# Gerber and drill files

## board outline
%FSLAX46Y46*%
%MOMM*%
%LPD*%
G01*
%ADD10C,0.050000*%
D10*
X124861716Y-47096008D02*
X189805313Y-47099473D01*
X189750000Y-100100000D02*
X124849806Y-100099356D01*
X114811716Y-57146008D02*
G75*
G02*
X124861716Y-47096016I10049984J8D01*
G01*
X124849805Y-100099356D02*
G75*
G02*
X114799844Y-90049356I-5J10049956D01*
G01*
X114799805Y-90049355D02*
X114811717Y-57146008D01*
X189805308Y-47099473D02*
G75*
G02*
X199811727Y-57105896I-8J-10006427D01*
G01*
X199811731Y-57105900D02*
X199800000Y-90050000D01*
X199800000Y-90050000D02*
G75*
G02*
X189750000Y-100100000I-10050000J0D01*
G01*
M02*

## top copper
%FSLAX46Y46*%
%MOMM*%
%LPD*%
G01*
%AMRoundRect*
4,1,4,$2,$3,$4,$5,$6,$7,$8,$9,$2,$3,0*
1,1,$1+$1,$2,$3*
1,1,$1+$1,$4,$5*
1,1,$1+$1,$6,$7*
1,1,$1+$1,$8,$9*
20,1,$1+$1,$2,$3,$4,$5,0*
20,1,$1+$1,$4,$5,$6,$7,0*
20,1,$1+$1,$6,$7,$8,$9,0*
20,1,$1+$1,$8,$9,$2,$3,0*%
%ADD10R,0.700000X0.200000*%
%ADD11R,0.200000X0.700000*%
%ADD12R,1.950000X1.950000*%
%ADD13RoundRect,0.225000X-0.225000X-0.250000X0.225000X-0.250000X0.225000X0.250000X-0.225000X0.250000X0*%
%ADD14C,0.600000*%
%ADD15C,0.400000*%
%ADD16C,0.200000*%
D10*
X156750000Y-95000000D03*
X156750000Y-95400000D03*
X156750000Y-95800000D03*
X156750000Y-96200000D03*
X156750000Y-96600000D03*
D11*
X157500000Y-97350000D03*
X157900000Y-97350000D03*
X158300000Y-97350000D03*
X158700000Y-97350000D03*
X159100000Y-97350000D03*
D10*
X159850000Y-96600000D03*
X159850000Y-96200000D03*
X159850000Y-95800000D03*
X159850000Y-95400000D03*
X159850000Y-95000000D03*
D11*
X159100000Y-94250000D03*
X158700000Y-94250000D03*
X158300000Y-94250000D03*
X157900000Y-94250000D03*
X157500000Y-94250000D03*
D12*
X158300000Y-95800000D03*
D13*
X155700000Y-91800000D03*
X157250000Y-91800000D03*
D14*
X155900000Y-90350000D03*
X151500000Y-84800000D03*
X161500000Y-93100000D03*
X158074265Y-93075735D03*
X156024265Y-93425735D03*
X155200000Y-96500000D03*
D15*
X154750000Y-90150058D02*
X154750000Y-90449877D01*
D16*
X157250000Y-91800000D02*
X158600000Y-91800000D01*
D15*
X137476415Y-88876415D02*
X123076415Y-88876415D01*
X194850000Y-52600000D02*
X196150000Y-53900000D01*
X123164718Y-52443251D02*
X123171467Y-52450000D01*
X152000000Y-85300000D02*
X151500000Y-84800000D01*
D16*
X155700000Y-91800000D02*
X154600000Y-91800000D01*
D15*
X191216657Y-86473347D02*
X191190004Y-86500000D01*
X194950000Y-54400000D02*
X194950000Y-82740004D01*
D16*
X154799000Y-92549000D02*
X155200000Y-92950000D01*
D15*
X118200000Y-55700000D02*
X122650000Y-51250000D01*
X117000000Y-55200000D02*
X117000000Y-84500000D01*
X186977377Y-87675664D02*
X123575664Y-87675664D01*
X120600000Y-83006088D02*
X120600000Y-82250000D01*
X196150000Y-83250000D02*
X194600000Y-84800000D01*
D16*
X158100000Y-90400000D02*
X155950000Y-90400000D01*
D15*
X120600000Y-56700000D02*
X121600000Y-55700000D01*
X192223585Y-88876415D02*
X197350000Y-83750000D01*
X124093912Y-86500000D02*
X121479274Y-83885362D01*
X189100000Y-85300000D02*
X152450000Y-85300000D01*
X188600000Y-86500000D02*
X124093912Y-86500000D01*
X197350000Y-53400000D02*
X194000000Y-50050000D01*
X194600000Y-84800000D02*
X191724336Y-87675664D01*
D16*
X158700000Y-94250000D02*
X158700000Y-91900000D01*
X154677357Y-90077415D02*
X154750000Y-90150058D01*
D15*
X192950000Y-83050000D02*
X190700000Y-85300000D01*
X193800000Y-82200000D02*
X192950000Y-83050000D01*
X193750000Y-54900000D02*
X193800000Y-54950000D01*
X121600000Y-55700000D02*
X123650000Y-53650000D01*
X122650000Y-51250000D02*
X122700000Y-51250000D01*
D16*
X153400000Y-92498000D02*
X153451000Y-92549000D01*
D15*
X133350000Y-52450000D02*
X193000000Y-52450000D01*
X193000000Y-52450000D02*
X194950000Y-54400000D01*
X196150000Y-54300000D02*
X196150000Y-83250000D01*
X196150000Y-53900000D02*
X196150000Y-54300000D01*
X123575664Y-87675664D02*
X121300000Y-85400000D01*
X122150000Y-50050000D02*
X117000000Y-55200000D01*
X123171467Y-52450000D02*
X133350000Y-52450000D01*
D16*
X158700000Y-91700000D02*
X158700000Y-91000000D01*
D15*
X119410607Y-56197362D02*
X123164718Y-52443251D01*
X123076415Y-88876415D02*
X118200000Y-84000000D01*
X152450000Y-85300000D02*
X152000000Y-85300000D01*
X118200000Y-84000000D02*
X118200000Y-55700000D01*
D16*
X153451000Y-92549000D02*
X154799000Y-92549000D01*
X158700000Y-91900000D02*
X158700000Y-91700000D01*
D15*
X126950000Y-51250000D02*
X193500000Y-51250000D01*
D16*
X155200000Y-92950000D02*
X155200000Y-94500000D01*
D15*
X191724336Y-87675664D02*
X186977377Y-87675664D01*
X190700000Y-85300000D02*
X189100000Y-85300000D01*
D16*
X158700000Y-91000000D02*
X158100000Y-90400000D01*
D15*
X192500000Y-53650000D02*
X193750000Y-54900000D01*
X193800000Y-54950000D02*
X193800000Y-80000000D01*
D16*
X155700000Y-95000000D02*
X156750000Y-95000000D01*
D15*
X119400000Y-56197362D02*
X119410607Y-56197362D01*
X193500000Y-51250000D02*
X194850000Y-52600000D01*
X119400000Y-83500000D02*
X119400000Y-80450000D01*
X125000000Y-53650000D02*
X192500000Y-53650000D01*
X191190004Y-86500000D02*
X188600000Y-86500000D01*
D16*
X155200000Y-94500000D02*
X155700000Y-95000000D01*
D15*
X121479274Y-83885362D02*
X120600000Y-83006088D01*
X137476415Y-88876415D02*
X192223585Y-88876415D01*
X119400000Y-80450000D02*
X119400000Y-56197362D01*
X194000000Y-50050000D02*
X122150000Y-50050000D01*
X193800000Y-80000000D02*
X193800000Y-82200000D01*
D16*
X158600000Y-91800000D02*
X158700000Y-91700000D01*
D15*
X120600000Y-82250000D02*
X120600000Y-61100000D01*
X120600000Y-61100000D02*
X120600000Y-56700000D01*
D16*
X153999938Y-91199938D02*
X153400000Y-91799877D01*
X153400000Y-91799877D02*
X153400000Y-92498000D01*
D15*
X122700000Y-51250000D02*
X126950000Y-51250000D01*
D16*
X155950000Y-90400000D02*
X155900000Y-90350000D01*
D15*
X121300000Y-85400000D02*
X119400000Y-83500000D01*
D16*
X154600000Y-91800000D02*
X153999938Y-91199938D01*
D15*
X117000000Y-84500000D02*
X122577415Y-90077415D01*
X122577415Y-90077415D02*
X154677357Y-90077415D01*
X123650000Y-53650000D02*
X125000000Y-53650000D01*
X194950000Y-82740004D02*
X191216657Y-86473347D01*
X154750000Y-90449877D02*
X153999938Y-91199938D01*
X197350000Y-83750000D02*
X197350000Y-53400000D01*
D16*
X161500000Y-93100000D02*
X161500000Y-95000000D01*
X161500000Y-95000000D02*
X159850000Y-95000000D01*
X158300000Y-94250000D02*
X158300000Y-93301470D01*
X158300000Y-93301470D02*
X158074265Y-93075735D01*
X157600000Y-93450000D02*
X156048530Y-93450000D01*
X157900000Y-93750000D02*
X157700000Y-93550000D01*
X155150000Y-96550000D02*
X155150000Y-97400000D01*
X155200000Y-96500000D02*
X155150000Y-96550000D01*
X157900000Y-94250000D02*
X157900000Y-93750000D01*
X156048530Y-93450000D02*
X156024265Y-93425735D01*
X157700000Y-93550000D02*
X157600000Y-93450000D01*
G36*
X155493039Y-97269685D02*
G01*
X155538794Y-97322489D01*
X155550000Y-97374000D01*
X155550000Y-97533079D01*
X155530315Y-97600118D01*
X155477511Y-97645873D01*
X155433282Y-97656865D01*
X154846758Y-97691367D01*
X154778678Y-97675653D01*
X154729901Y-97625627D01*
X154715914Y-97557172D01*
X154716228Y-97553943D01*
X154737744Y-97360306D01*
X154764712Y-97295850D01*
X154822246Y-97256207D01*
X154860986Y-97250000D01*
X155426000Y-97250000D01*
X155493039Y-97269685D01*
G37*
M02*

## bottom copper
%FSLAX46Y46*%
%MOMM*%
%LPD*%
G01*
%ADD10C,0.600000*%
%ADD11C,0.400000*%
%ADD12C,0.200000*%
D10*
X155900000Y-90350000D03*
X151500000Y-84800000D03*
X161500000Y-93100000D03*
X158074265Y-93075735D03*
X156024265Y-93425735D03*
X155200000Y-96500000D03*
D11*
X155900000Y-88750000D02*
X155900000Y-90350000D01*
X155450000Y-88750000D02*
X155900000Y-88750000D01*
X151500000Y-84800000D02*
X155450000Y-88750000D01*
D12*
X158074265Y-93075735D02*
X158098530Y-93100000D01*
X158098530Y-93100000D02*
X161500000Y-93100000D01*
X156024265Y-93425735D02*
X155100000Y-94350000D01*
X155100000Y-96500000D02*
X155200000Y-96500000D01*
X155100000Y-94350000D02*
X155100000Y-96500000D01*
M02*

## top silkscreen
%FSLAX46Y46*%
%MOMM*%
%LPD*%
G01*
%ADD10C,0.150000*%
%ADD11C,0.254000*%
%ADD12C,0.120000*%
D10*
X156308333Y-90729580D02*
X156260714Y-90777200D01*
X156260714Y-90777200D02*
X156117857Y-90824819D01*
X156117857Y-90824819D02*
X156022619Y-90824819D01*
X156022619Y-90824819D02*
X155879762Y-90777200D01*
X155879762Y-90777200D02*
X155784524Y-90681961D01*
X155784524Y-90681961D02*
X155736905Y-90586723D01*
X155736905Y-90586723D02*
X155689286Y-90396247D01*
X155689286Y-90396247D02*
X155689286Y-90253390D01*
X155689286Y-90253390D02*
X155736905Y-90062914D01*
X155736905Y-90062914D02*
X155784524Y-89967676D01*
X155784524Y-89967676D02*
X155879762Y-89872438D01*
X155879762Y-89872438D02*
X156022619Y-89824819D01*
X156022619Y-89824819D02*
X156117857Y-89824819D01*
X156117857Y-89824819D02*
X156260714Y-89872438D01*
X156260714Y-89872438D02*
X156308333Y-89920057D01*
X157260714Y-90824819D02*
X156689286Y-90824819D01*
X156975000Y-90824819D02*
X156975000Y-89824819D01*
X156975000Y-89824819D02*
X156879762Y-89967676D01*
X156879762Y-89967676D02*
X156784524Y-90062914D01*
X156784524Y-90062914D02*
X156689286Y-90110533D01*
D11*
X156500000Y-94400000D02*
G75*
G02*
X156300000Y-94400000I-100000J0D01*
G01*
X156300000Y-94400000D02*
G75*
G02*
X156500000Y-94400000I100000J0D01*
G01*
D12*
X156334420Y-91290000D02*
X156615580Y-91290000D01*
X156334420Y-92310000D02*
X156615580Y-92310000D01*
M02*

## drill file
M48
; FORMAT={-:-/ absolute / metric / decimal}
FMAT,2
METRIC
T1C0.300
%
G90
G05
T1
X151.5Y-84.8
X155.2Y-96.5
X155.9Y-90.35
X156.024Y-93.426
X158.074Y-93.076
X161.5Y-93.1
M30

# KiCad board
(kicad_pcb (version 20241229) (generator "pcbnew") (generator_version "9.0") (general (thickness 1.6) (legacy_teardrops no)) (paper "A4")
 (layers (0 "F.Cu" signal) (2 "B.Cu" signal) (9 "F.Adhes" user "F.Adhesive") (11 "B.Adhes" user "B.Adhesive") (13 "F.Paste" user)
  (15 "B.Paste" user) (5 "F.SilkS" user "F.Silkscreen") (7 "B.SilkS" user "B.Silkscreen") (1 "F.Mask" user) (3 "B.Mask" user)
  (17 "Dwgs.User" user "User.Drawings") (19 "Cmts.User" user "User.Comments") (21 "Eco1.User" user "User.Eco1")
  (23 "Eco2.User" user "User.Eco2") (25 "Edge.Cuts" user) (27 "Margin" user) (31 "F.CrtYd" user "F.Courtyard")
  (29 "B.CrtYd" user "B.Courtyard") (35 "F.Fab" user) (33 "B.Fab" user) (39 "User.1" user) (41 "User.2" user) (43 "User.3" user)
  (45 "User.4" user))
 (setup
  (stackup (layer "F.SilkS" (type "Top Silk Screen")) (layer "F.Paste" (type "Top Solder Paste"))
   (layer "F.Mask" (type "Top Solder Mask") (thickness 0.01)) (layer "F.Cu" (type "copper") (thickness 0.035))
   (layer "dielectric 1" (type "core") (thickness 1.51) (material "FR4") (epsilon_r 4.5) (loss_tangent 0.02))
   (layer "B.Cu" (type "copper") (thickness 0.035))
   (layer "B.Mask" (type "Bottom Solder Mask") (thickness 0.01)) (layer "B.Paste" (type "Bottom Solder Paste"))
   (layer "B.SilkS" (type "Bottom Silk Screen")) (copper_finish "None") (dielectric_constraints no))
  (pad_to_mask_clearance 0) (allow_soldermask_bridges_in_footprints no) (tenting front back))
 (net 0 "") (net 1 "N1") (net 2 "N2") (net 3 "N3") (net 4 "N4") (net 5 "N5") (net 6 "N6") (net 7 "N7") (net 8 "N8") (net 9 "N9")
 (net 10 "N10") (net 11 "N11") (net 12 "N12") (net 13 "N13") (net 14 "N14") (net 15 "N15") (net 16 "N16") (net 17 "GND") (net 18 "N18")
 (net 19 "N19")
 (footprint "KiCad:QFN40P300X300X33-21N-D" (layer "F.Cu") (at 158.3 95.8)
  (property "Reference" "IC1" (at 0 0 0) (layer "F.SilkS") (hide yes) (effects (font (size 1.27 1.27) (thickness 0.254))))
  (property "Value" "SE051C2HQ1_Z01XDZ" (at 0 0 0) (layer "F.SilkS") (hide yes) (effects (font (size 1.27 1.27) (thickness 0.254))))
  (fp_circle (center -1.9 -1.4) (end -1.8 -1.4) (stroke (width 0.254) (type solid)) (fill no) (layer "F.SilkS"))
  (pad "1" smd rect (at -1.55 -0.8 90) (size 0.2 0.7) (layers "F.Cu" "F.Mask" "F.Paste") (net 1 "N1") (solder_mask_margin 0.04)
   (thermal_bridge_angle 45))
  (pad "2" smd rect (at -1.55 -0.4 90) (size 0.2 0.7) (layers "F.Cu" "F.Mask" "F.Paste") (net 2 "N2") (solder_mask_margin 0.04)
   (thermal_bridge_angle 45))
  (pad "3" smd rect (at -1.55 0 90) (size 0.2 0.7) (layers "F.Cu" "F.Mask" "F.Paste") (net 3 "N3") (solder_mask_margin 0.04)
   (thermal_bridge_angle 45))
  (pad "4" smd rect (at -1.55 0.4 90) (size 0.2 0.7) (layers "F.Cu" "F.Mask" "F.Paste") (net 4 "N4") (solder_mask_margin 0.04)
   (thermal_bridge_angle 45))
  (pad "5" smd rect (at -1.55 0.8 90) (size 0.2 0.7) (layers "F.Cu" "F.Mask" "F.Paste") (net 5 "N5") (solder_mask_margin 0.04)
   (thermal_bridge_angle 45))
  (pad "6" smd rect (at -0.8 1.55) (size 0.2 0.7) (layers "F.Cu" "F.Mask" "F.Paste") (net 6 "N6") (solder_mask_margin 0.04)
   (thermal_bridge_angle 45))
  (pad "7" smd rect (at -0.4 1.55) (size 0.2 0.7) (layers "F.Cu" "F.Mask" "F.Paste") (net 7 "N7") (solder_mask_margin 0.04)
   (thermal_bridge_angle 45))
  (pad "8" smd rect (at 0 1.55) (size 0.2 0.7) (layers "F.Cu" "F.Mask" "F.Paste") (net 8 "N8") (solder_mask_margin 0.04)
   (thermal_bridge_angle 45))
  (pad "9" smd rect (at 0.4 1.55) (size 0.2 0.7) (layers "F.Cu" "F.Mask" "F.Paste") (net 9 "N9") (solder_mask_margin 0.04)
   (thermal_bridge_angle 45))
  (pad "10" smd rect (at 0.8 1.55) (size 0.2 0.7) (layers "F.Cu" "F.Mask" "F.Paste") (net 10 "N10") (solder_mask_margin 0.04)
   (thermal_bridge_angle 45))
  (pad "11" smd rect (at 1.55 0.8 90) (size 0.2 0.7) (layers "F.Cu" "F.Mask" "F.Paste") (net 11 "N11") (solder_mask_margin 0.04)
   (thermal_bridge_angle 45))
  (pad "12" smd rect (at 1.55 0.4 90) (size 0.2 0.7) (layers "F.Cu" "F.Mask" "F.Paste") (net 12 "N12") (solder_mask_margin 0.04)
   (thermal_bridge_angle 45))
  (pad "13" smd rect (at 1.55 0 90) (size 0.2 0.7) (layers "F.Cu" "F.Mask" "F.Paste") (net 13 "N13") (solder_mask_margin 0.04)
   (thermal_bridge_angle 45))
  (pad "14" smd rect (at 1.55 -0.4 90) (size 0.2 0.7) (layers "F.Cu" "F.Mask" "F.Paste") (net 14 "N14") (solder_mask_margin 0.04)
   (thermal_bridge_angle 45))
  (pad "15" smd rect (at 1.55 -0.8 90) (size 0.2 0.7) (layers "F.Cu" "F.Mask" "F.Paste") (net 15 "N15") (solder_mask_margin 0.04)
   (thermal_bridge_angle 45))
  (pad "16" smd rect (at 0.8 -1.55) (size 0.2 0.7) (layers "F.Cu" "F.Mask" "F.Paste") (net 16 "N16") (solder_mask_margin 0.04)
   (thermal_bridge_angle 45))
  (pad "17" smd rect (at 0.4 -1.55) (size 0.2 0.7) (layers "F.Cu" "F.Mask" "F.Paste") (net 1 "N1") (solder_mask_margin 0.04)
   (thermal_bridge_angle 45))
  (pad "18" smd rect (at 0 -1.55) (size 0.2 0.7) (layers "F.Cu" "F.Mask" "F.Paste") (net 15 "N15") (solder_mask_margin 0.04)
   (thermal_bridge_angle 45))
  (pad "19" smd rect (at -0.4 -1.55) (size 0.2 0.7) (layers "F.Cu" "F.Mask" "F.Paste") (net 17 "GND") (solder_mask_margin 0.04)
   (thermal_bridge_angle 45))
  (pad "20" smd rect (at -0.8 -1.55) (size 0.2 0.7) (layers "F.Cu" "F.Mask" "F.Paste") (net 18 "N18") (solder_mask_margin 0.04)
   (thermal_bridge_angle 45))
  (pad "21" smd rect (at 0 0) (size 1.95 1.95) (layers "F.Cu" "F.Mask" "F.Paste") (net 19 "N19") (thermal_bridge_angle 45)))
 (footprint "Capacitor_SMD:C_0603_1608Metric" (layer "F.Cu") (at 156.475 91.8)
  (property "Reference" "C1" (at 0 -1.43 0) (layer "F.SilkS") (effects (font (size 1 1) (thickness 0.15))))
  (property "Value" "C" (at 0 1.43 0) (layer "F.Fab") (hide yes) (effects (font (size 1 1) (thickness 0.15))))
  (fp_line (start -0.14058 -0.51) (end 0.14058 -0.51) (stroke (width 0.12) (type solid)) (layer "F.SilkS"))
  (fp_line (start -0.14058 0.51) (end 0.14058 0.51) (stroke (width 0.12) (type solid)) (layer "F.SilkS"))
  (pad "1" smd roundrect (at -0.775 0) (size 0.9 0.95) (layers "F.Cu" "F.Mask" "F.Paste") (roundrect_rratio 0.25) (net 1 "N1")
   (solder_mask_margin 0.04))
  (pad "2" smd roundrect (at 0.775 0) (size 0.9 0.95) (layers "F.Cu" "F.Mask" "F.Paste") (roundrect_rratio 0.25) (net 1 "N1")
   (solder_mask_margin 0.04)))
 (gr_line (start 124.861716 47.096008) (end 189.805313 47.099473) (stroke (width 0.05) (type default)) (layer "Edge.Cuts"))
 (gr_line (start 189.75 100.1) (end 124.849806 100.099356) (stroke (width 0.05) (type default)) (layer "Edge.Cuts"))
 (gr_arc (start 114.811716 57.146008) (mid 117.755293 50.039585) (end 124.861716 47.096008) (stroke (width 0.05) (type default))
  (layer "Edge.Cuts"))
 (gr_arc (start 124.849805 100.099356) (mid 117.743382 97.155779) (end 114.799805 90.049356) (stroke (width 0.05) (type default))
  (layer "Edge.Cuts"))
 (gr_line (start 114.799805 90.049355) (end 114.811717 57.146008) (stroke (width 0.05) (type default)) (layer "Edge.Cuts"))
 (gr_arc (start 189.805308 47.099473) (mid 196.880918 50.030286) (end 199.811731 57.105896) (stroke (width 0.05) (type default))
  (layer "Edge.Cuts"))
 (gr_line (start 199.811731 57.1059) (end 199.8 90.05) (stroke (width 0.05) (type default)) (layer "Edge.Cuts"))
 (gr_arc (start 199.8 90.05) (mid 196.856423 97.156423) (end 189.75 100.1) (stroke (width 0.05) (type default)) (layer "Edge.Cuts"))
 (segment (start 154.75 90.150058) (end 154.75 90.449877) (width 0.4) (layer "F.Cu") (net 1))
 (segment (start 157.25 91.8) (end 158.6 91.8) (width 0.2) (layer "F.Cu") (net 1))
 (segment (start 137.476415 88.876415) (end 123.076415 88.876415) (width 0.4) (layer "F.Cu") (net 1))
 (segment (start 194.85 52.6) (end 196.15 53.9) (width 0.4) (layer "F.Cu") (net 1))
 (segment (start 123.164718 52.443251) (end 123.171467 52.45) (width 0.4) (layer "F.Cu") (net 1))
 (segment (start 152 85.3) (end 151.5 84.8) (width 0.4) (layer "F.Cu") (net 1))
 (segment (start 155.7 91.8) (end 154.6 91.8) (width 0.2) (layer "F.Cu") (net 1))
 (segment (start 191.216657 86.473347) (end 191.190004 86.5) (width 0.4) (layer "F.Cu") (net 1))
 (segment (start 194.95 54.4) (end 194.95 82.740004) (width 0.4) (layer "F.Cu") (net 1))
 (segment (start 154.799 92.549) (end 155.2 92.95) (width 0.2) (layer "F.Cu") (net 1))
 (segment (start 118.2 55.7) (end 122.65 51.25) (width 0.4) (layer "F.Cu") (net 1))
 (segment (start 117 55.2) (end 117 84.5) (width 0.4) (layer "F.Cu") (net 1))
 (segment (start 186.977377 87.675664) (end 123.575664 87.675664) (width 0.4) (layer "F.Cu") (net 1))
 (segment (start 120.6 83.006088) (end 120.6 82.25) (width 0.4) (layer "F.Cu") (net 1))
 (segment (start 196.15 83.25) (end 194.6 84.8) (width 0.4) (layer "F.Cu") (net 1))
 (segment (start 158.1 90.4) (end 155.95 90.4) (width 0.2) (layer "F.Cu") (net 1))
 (segment (start 120.6 56.7) (end 121.6 55.7) (width 0.4) (layer "F.Cu") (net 1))
 (segment (start 192.223585 88.876415) (end 197.35 83.75) (width 0.4) (layer "F.Cu") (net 1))
 (segment (start 124.093912 86.5) (end 121.479274 83.885362) (width 0.4) (layer "F.Cu") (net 1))
 (segment (start 189.1 85.3) (end 152.45 85.3) (width 0.4) (layer "F.Cu") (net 1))
 (segment (start 188.6 86.5) (end 124.093912 86.5) (width 0.4) (layer "F.Cu") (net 1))
 (segment (start 197.35 53.4) (end 194 50.05) (width 0.4) (layer "F.Cu") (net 1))
 (segment (start 194.6 84.8) (end 191.724336 87.675664) (width 0.4) (layer "F.Cu") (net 1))
 (segment (start 158.7 94.25) (end 158.7 91.9) (width 0.2) (layer "F.Cu") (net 1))
 (segment (start 154.677357 90.077415) (end 154.75 90.150058) (width 0.2) (layer "F.Cu") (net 1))
 (segment (start 192.95 83.05) (end 190.7 85.3) (width 0.4) (layer "F.Cu") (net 1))
 (segment (start 193.8 82.2) (end 192.95 83.05) (width 0.4) (layer "F.Cu") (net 1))
 (segment (start 193.75 54.9) (end 193.8 54.95) (width 0.4) (layer "F.Cu") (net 1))
 (segment (start 121.6 55.7) (end 123.65 53.65) (width 0.4) (layer "F.Cu") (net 1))
 (segment (start 122.65 51.25) (end 122.7 51.25) (width 0.4) (layer "F.Cu") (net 1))
 (segment (start 153.4 92.498) (end 153.451 92.549) (width 0.2) (layer "F.Cu") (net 1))
 (segment (start 133.35 52.45) (end 193 52.45) (width 0.4) (layer "F.Cu") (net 1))
 (segment (start 193 52.45) (end 194.95 54.4) (width 0.4) (layer "F.Cu") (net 1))
 (segment (start 196.15 54.3) (end 196.15 83.25) (width 0.4) (layer "F.Cu") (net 1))
 (segment (start 196.15 53.9) (end 196.15 54.3) (width 0.4) (layer "F.Cu") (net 1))
 (segment (start 123.575664 87.675664) (end 121.3 85.4) (width 0.4) (layer "F.Cu") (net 1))
 (segment (start 122.15 50.05) (end 117 55.2) (width 0.4) (layer "F.Cu") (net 1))
 (segment (start 123.171467 52.45) (end 133.35 52.45) (width 0.4) (layer "F.Cu") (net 1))
 (segment (start 158.7 91.7) (end 158.7 91) (width 0.2) (layer "F.Cu") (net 1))
 (segment (start 119.410607 56.197362) (end 123.164718 52.443251) (width 0.4) (layer "F.Cu") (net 1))
 (segment (start 123.076415 88.876415) (end 118.2 84) (width 0.4) (layer "F.Cu") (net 1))
 (segment (start 152.45 85.3) (end 152 85.3) (width 0.4) (layer "F.Cu") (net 1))
 (segment (start 118.2 84) (end 118.2 55.7) (width 0.4) (layer "F.Cu") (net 1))
 (segment (start 153.451 92.549) (end 154.799 92.549) (width 0.2) (layer "F.Cu") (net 1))
 (segment (start 158.7 91.9) (end 158.7 91.7) (width 0.2) (layer "F.Cu") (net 1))
 (segment (start 126.95 51.25) (end 193.5 51.25) (width 0.4) (layer "F.Cu") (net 1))
 (segment (start 155.2 92.95) (end 155.2 94.5) (width 0.2) (layer "F.Cu") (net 1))
 (segment (start 191.724336 87.675664) (end 186.977377 87.675664) (width 0.4) (layer "F.Cu") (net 1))
 (segment (start 190.7 85.3) (end 189.1 85.3) (width 0.4) (layer "F.Cu") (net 1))
 (segment (start 158.7 91) (end 158.1 90.4) (width 0.2) (layer "F.Cu") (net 1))
 (segment (start 192.5 53.65) (end 193.75 54.9) (width 0.4) (layer "F.Cu") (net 1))
 (segment (start 193.8 54.95) (end 193.8 80) (width 0.4) (layer "F.Cu") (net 1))
 (segment (start 155.7 95) (end 156.75 95) (width 0.2) (layer "F.Cu") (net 1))
 (segment (start 119.4 56.197362) (end 119.410607 56.197362) (width 0.4) (layer "F.Cu") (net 1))
 (segment (start 193.5 51.25) (end 194.85 52.6) (width 0.4) (layer "F.Cu") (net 1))
 (segment (start 119.4 83.5) (end 119.4 80.45) (width 0.4) (layer "F.Cu") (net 1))
 (segment (start 125 53.65) (end 192.5 53.65) (width 0.4) (layer "F.Cu") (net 1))
 (segment (start 191.190004 86.5) (end 188.6 86.5) (width 0.4) (layer "F.Cu") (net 1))
 (segment (start 155.2 94.5) (end 155.7 95) (width 0.2) (layer "F.Cu") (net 1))
 (segment (start 121.479274 83.885362) (end 120.6 83.006088) (width 0.4) (layer "F.Cu") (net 1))
 (segment (start 137.476415 88.876415) (end 192.223585 88.876415) (width 0.4) (layer "F.Cu") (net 1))
 (segment (start 119.4 80.45) (end 119.4 56.197362) (width 0.4) (layer "F.Cu") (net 1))
 (segment (start 194 50.05) (end 122.15 50.05) (width 0.4) (layer "F.Cu") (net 1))
 (segment (start 193.8 80) (end 193.8 82.2) (width 0.4) (layer "F.Cu") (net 1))
 (segment (start 158.6 91.8) (end 158.7 91.7) (width 0.2) (layer "F.Cu") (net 1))
 (segment (start 120.6 82.25) (end 120.6 61.1) (width 0.4) (layer "F.Cu") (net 1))
 (segment (start 120.6 61.1) (end 120.6 56.7) (width 0.4) (layer "F.Cu") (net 1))
 (segment (start 153.999938 91.199938) (end 153.4 91.799877) (width 0.2) (layer "F.Cu") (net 1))
 (segment (start 153.4 91.799877) (end 153.4 92.498) (width 0.2) (layer "F.Cu") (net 1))
 (segment (start 122.7 51.25) (end 126.95 51.25) (width 0.4) (layer "F.Cu") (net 1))
 (segment (start 155.95 90.4) (end 155.9 90.35) (width 0.2) (layer "F.Cu") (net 1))
 (segment (start 121.3 85.4) (end 119.4 83.5) (width 0.4) (layer "F.Cu") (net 1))
 (segment (start 154.6 91.8) (end 153.999938 91.199938) (width 0.2) (layer "F.Cu") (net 1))
 (segment (start 117 84.5) (end 122.577415 90.077415) (width 0.4) (layer "F.Cu") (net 1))
 (segment (start 122.577415 90.077415) (end 154.677357 90.077415) (width 0.4) (layer "F.Cu") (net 1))
 (segment (start 123.65 53.65) (end 125 53.65) (width 0.4) (layer "F.Cu") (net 1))
 (segment (start 194.95 82.740004) (end 191.216657 86.473347) (width 0.4) (layer "F.Cu") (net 1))
 (segment (start 154.75 90.449877) (end 153.999938 91.199938) (width 0.4) (layer "F.Cu") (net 1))
 (segment (start 197.35 83.75) (end 197.35 53.4) (width 0.4) (layer "F.Cu") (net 1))
 (via (at 155.9 90.35) (size 0.6) (drill 0.3) (layers "F.Cu" "B.Cu") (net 1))
 (via (at 151.5 84.8) (size 0.6) (drill 0.3) (layers "F.Cu" "B.Cu") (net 1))
 (segment (start 155.9 88.75) (end 155.9 90.35) (width 0.4) (layer "B.Cu") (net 1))
 (segment (start 155.45 88.75) (end 155.9 88.75) (width 0.4) (layer "B.Cu") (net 1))
 (segment (start 151.5 84.8) (end 155.45 88.75) (width 0.4) (layer "B.Cu") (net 1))
 (segment (start 161.5 93.1) (end 161.5 95) (width 0.2) (layer "F.Cu") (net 15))
 (segment (start 161.5 95) (end 159.85 95) (width 0.2) (layer "F.Cu") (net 15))
 (segment (start 158.3 94.25) (end 158.3 93.30147) (width 0.2) (layer "F.Cu") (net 15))
 (segment (start 158.3 93.30147) (end 158.074265 93.075735) (width 0.2) (layer "F.Cu") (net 15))
 (via (at 161.5 93.1) (size 0.6) (drill 0.3) (layers "F.Cu" "B.Cu") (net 15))
 (via (at 158.074265 93.075735) (size 0.6) (drill 0.3) (layers "F.Cu" "B.Cu") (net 15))
 (segment (start 158.074265 93.075735) (end 158.09853 93.1) (width 0.2) (layer "B.Cu") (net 15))
 (segment (start 158.09853 93.1) (end 161.5 93.1) (width 0.2) (layer "B.Cu") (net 15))
 (segment (start 157.6 93.45) (end 156.04853 93.45) (width 0.2) (layer "F.Cu") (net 17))
 (segment (start 157.9 93.75) (end 157.7 93.55) (width 0.2) (layer "F.Cu") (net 17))
 (segment (start 155.15 96.55) (end 155.15 97.4) (width 0.2) (layer "F.Cu") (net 17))
 (segment (start 155.2 96.5) (end 155.15 96.55) (width 0.2) (layer "F.Cu") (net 17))
 (segment (start 157.9 94.25) (end 157.9 93.75) (width 0.2) (layer "F.Cu") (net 17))
 (segment (start 156.04853 93.45) (end 156.024265 93.425735) (width 0.2) (layer "F.Cu") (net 17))
 (segment (start 157.7 93.55) (end 157.6 93.45) (width 0.2) (layer "F.Cu") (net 17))
 (via (at 156.024265 93.425735) (size 0.6) (drill 0.3) (layers "F.Cu" "B.Cu") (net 17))
 (via (at 155.2 96.5) (size 0.6) (drill 0.3) (layers "F.Cu" "B.Cu") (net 17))
 (segment (start 156.024265 93.425735) (end 155.1 94.35) (width 0.2) (layer "B.Cu") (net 17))
 (segment (start 155.1 96.5) (end 155.2 96.5) (width 0.2) (layer "B.Cu") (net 17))
 (segment (start 155.1 94.35) (end 155.1 96.5) (width 0.2) (layer "B.Cu") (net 17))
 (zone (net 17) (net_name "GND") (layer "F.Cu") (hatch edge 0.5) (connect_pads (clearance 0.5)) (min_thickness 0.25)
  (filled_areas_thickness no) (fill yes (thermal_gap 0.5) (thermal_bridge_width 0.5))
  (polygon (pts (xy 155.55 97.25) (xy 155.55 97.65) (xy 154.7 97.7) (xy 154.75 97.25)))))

